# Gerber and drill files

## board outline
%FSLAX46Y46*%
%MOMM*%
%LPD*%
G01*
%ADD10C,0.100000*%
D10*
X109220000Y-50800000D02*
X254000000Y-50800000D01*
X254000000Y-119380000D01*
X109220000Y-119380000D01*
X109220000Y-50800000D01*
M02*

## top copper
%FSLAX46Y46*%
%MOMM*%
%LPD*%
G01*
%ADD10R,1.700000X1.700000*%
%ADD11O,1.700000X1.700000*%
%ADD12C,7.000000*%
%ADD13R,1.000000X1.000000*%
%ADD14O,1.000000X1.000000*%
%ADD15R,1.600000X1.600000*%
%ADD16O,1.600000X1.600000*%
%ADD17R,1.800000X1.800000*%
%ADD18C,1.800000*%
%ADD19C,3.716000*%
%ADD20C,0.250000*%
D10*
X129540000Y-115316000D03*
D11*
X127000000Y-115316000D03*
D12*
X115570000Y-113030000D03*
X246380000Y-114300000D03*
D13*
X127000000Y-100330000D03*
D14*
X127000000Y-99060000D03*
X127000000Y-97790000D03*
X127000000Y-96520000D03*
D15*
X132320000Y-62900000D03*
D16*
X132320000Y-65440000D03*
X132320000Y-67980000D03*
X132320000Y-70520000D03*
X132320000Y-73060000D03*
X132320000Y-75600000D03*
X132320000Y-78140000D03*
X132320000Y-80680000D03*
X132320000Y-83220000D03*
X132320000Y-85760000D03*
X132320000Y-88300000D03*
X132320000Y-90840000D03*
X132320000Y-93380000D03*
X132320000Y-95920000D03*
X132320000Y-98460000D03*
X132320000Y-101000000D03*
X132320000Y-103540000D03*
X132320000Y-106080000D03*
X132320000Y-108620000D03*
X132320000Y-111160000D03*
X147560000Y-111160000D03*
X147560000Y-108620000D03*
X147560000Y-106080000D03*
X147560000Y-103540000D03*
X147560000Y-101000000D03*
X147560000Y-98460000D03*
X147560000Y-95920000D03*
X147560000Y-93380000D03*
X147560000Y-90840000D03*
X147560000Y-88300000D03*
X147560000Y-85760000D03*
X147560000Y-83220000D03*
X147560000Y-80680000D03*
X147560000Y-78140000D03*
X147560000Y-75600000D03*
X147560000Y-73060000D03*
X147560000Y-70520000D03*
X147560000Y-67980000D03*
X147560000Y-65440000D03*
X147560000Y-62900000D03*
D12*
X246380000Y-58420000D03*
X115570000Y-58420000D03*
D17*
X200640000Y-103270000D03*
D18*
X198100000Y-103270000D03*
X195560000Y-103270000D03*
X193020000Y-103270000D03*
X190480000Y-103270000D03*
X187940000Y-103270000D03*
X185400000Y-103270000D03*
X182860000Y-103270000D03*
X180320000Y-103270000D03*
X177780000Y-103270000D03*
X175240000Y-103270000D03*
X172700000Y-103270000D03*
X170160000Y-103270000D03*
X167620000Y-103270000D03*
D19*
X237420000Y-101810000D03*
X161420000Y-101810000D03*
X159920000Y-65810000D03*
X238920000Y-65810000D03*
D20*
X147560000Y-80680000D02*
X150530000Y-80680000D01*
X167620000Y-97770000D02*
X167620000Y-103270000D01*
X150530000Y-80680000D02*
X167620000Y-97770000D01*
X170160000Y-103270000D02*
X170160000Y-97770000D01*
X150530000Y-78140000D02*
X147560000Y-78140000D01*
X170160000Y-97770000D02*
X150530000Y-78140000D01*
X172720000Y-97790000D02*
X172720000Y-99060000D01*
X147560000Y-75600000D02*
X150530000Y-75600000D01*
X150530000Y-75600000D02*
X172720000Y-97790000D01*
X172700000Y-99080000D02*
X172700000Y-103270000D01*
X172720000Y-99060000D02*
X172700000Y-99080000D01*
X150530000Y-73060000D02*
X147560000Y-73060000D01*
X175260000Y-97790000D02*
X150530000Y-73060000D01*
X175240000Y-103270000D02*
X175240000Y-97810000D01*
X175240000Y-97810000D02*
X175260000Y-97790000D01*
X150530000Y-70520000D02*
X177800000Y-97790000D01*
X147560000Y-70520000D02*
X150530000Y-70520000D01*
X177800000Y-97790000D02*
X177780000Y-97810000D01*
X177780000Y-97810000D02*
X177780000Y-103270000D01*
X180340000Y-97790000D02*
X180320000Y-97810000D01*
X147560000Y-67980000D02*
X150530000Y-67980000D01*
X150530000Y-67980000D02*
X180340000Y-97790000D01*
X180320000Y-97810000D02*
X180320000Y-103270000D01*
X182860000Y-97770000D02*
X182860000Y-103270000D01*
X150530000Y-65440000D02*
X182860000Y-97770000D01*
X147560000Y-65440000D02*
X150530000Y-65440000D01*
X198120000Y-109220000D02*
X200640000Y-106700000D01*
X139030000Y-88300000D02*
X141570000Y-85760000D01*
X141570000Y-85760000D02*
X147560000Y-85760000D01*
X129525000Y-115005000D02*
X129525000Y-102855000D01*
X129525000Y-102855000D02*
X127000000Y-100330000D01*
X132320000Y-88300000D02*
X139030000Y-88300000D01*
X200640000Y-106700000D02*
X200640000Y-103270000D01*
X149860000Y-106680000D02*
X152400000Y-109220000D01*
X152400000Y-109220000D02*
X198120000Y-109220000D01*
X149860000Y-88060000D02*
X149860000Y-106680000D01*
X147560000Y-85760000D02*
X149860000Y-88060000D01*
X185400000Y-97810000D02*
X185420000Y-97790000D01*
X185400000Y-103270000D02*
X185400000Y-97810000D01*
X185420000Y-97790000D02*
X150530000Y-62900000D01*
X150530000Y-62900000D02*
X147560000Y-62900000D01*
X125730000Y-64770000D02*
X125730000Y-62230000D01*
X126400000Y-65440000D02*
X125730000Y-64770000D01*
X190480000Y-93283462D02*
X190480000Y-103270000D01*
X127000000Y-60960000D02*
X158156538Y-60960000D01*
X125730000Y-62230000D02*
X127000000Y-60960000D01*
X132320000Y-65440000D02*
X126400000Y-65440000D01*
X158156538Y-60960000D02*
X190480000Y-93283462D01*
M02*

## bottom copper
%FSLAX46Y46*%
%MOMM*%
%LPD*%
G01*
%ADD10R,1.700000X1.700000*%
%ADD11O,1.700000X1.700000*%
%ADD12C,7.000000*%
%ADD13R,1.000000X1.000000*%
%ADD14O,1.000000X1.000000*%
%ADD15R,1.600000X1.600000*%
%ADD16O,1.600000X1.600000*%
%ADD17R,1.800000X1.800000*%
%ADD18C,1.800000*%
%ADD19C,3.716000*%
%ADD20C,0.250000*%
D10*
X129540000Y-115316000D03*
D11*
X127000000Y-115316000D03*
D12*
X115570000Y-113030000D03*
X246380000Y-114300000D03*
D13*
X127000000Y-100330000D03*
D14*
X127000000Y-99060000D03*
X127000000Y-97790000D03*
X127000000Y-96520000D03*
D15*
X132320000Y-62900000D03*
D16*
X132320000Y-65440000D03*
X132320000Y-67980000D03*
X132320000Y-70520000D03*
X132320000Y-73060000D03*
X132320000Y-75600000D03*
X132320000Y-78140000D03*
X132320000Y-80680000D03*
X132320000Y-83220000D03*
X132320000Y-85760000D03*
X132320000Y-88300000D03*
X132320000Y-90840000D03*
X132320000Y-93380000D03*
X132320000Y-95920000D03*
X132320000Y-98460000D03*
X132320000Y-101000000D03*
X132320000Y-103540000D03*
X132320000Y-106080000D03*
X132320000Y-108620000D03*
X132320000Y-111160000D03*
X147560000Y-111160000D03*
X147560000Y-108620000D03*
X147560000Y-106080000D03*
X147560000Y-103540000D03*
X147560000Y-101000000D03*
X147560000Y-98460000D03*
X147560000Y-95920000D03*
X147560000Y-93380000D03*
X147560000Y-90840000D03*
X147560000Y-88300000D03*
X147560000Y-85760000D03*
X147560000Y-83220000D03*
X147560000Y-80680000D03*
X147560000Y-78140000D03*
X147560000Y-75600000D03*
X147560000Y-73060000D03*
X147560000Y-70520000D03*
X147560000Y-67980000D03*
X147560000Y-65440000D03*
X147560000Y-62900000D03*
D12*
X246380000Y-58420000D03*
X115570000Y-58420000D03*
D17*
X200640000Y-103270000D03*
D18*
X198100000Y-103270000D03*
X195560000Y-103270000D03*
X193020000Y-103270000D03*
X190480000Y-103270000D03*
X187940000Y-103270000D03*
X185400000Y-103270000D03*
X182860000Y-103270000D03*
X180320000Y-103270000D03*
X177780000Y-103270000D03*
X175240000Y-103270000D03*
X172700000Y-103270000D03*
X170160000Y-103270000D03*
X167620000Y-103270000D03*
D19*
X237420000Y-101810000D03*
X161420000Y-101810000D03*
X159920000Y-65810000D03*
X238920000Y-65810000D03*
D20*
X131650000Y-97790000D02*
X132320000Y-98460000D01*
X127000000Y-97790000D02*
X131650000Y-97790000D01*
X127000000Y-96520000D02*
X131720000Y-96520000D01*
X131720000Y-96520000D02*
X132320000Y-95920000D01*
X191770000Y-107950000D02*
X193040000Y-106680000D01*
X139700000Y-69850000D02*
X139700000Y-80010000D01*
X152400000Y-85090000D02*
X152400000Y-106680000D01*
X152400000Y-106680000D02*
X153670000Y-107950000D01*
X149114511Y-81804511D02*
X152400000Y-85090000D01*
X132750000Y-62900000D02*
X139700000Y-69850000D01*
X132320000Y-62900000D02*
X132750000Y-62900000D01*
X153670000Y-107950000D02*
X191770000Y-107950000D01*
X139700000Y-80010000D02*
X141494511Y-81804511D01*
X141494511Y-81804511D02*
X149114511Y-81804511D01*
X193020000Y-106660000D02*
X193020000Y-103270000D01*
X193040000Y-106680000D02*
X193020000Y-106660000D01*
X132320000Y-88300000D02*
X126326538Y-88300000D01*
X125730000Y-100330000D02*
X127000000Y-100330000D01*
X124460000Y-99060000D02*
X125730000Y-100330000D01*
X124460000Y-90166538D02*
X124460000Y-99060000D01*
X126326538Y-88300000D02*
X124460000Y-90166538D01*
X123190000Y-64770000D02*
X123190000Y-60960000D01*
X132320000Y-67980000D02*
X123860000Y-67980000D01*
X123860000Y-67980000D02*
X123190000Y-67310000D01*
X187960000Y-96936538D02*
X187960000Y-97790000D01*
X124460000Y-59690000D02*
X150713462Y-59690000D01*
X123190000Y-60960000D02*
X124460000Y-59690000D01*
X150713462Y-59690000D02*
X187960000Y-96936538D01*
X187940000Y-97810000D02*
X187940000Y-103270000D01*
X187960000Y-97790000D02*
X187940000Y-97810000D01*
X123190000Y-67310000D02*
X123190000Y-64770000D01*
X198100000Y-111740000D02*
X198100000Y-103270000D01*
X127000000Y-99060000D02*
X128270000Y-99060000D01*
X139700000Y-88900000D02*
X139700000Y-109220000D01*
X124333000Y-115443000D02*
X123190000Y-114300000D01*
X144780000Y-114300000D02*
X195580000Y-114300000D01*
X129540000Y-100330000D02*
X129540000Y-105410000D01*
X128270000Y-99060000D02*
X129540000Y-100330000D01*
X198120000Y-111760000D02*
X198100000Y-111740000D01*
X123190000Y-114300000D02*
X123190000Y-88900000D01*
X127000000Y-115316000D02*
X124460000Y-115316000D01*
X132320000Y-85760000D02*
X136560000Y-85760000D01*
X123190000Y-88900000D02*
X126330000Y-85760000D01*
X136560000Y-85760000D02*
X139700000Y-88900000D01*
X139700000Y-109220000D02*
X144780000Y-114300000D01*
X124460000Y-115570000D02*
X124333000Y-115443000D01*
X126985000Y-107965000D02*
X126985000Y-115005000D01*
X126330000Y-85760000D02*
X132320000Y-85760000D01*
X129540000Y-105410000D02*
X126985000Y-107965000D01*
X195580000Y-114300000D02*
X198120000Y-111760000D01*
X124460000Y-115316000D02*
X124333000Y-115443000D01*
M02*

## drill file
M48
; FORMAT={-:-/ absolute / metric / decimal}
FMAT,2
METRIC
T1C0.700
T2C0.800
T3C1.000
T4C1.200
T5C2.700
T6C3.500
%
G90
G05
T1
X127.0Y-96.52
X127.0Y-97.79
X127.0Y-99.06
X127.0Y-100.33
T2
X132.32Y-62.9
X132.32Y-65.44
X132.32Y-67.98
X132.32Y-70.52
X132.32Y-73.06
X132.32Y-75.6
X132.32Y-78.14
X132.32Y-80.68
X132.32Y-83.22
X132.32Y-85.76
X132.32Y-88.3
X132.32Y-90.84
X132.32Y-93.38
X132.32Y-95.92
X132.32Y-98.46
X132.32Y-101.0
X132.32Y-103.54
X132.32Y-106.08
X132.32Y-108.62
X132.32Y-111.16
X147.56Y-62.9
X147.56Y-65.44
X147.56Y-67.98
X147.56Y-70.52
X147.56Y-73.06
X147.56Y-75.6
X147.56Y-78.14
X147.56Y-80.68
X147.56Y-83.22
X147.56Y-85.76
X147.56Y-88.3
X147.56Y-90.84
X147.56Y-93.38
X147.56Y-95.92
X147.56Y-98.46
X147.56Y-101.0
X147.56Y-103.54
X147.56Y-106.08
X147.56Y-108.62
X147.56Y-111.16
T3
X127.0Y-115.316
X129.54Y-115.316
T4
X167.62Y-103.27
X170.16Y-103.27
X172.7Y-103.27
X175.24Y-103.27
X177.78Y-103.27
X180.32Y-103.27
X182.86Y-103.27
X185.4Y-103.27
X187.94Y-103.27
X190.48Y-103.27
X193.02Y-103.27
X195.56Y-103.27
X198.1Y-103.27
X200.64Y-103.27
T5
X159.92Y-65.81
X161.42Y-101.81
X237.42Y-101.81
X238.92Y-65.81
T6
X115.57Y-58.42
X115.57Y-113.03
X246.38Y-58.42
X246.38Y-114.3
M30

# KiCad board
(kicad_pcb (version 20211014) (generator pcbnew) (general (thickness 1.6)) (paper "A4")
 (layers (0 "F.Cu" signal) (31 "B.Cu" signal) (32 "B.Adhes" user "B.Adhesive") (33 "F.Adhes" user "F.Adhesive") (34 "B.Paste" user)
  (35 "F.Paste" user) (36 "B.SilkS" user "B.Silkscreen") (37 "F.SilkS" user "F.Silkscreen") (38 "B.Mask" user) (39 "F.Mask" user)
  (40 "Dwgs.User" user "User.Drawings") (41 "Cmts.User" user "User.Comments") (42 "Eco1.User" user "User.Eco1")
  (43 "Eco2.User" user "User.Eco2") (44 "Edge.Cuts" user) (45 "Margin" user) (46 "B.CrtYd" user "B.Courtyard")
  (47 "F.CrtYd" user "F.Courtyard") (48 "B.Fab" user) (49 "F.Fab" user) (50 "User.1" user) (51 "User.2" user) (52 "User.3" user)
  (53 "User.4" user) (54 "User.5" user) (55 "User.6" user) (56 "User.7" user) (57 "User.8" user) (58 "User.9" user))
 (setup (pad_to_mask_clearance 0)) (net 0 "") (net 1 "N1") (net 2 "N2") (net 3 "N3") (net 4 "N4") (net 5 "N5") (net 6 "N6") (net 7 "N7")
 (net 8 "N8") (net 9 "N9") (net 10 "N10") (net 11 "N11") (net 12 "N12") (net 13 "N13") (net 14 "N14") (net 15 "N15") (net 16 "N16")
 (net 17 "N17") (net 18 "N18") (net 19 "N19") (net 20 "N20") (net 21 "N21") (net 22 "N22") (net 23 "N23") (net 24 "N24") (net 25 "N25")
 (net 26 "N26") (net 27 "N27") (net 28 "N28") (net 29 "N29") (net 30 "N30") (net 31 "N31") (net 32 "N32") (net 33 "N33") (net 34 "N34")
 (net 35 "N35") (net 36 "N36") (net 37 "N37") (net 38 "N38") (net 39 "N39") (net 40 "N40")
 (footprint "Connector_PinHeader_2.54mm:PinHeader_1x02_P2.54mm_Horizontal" (layer "F.Cu") (at 129.54 115.316 -90)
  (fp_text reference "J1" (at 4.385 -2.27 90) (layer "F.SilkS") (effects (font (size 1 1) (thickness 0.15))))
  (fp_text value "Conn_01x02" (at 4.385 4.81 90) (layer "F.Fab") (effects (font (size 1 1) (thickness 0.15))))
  (pad "1" thru_hole rect (at 0 0 270) (size 1.7 1.7) (drill 1) (layers *.Cu *.Mask) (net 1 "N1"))
  (pad "2" thru_hole oval (at 0 2.54 270) (size 1.7 1.7) (drill 1) (layers *.Cu *.Mask) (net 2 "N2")))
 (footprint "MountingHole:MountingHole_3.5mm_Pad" (layer "F.Cu") (at 115.57 113.03)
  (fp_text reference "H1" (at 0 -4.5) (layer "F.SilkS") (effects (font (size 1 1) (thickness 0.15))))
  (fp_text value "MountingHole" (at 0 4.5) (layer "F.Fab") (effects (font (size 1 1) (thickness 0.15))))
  (pad "1" thru_hole circle (at 0 0) (size 7 7) (drill 3.5) (layers *.Cu *.Mask)))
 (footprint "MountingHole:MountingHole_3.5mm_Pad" (layer "F.Cu") (at 246.38 114.3)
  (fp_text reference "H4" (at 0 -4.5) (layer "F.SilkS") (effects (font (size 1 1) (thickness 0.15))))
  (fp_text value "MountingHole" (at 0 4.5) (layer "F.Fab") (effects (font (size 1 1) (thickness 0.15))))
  (pad "1" thru_hole circle (at 0 0) (size 7 7) (drill 3.5) (layers *.Cu *.Mask)))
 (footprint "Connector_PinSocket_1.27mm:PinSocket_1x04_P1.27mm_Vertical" (layer "F.Cu") (at 127 100.33 180)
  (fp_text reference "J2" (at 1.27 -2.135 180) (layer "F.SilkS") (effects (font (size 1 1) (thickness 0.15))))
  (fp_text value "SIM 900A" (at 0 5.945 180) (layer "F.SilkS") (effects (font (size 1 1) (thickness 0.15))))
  (pad "1" thru_hole rect (at 0 0 180) (size 1 1) (drill 0.7) (layers *.Cu *.Mask) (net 1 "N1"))
  (pad "2" thru_hole oval (at 0 1.27 180) (size 1 1) (drill 0.7) (layers *.Cu *.Mask) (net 2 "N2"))
  (pad "3" thru_hole oval (at 0 2.54 180) (size 1 1) (drill 0.7) (layers *.Cu *.Mask) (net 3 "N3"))
  (pad "4" thru_hole oval (at 0 3.81 180) (size 1 1) (drill 0.7) (layers *.Cu *.Mask) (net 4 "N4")))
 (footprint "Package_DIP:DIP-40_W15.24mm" (layer "F.Cu") (at 132.32 62.9)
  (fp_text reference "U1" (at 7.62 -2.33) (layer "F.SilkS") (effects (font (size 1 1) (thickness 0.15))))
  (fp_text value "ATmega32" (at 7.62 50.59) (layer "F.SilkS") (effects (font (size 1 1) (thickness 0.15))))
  (pad "1" thru_hole rect (at 0 0) (size 1.6 1.6) (drill 0.8) (layers *.Cu *.Mask) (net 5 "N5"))
  (pad "2" thru_hole oval (at 0 2.54) (size 1.6 1.6) (drill 0.8) (layers *.Cu *.Mask) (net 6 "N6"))
  (pad "3" thru_hole oval (at 0 5.08) (size 1.6 1.6) (drill 0.8) (layers *.Cu *.Mask) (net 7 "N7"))
  (pad "4" thru_hole oval (at 0 7.62) (size 1.6 1.6) (drill 0.8) (layers *.Cu *.Mask) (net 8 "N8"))
  (pad "5" thru_hole oval (at 0 10.16) (size 1.6 1.6) (drill 0.8) (layers *.Cu *.Mask) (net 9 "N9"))
  (pad "6" thru_hole oval (at 0 12.7) (size 1.6 1.6) (drill 0.8) (layers *.Cu *.Mask) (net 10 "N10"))
  (pad "7" thru_hole oval (at 0 15.24) (size 1.6 1.6) (drill 0.8) (layers *.Cu *.Mask) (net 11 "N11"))
  (pad "8" thru_hole oval (at 0 17.78) (size 1.6 1.6) (drill 0.8) (layers *.Cu *.Mask) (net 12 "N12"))
  (pad "9" thru_hole oval (at 0 20.32) (size 1.6 1.6) (drill 0.8) (layers *.Cu *.Mask) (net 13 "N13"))
  (pad "10" thru_hole oval (at 0 22.86) (size 1.6 1.6) (drill 0.8) (layers *.Cu *.Mask) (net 2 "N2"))
  (pad "11" thru_hole oval (at 0 25.4) (size 1.6 1.6) (drill 0.8) (layers *.Cu *.Mask) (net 1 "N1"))
  (pad "12" thru_hole oval (at 0 27.94) (size 1.6 1.6) (drill 0.8) (layers *.Cu *.Mask) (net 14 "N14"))
  (pad "13" thru_hole oval (at 0 30.48) (size 1.6 1.6) (drill 0.8) (layers *.Cu *.Mask) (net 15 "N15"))
  (pad "14" thru_hole oval (at 0 33.02) (size 1.6 1.6) (drill 0.8) (layers *.Cu *.Mask) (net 4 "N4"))
  (pad "15" thru_hole oval (at 0 35.56) (size 1.6 1.6) (drill 0.8) (layers *.Cu *.Mask) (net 3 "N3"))
  (pad "16" thru_hole oval (at 0 38.1) (size 1.6 1.6) (drill 0.8) (layers *.Cu *.Mask) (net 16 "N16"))
  (pad "17" thru_hole oval (at 0 40.64) (size 1.6 1.6) (drill 0.8) (layers *.Cu *.Mask) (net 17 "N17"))
  (pad "18" thru_hole oval (at 0 43.18) (size 1.6 1.6) (drill 0.8) (layers *.Cu *.Mask) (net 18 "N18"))
  (pad "19" thru_hole oval (at 0 45.72) (size 1.6 1.6) (drill 0.8) (layers *.Cu *.Mask) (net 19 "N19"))
  (pad "20" thru_hole oval (at 0 48.26) (size 1.6 1.6) (drill 0.8) (layers *.Cu *.Mask) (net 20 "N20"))
  (pad "21" thru_hole oval (at 15.24 48.26) (size 1.6 1.6) (drill 0.8) (layers *.Cu *.Mask) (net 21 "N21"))
  (pad "22" thru_hole oval (at 15.24 45.72) (size 1.6 1.6) (drill 0.8) (layers *.Cu *.Mask) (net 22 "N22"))
  (pad "23" thru_hole oval (at 15.24 43.18) (size 1.6 1.6) (drill 0.8) (layers *.Cu *.Mask) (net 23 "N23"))
  (pad "24" thru_hole oval (at 15.24 40.64) (size 1.6 1.6) (drill 0.8) (layers *.Cu *.Mask) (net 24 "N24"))
  (pad "25" thru_hole oval (at 15.24 38.1) (size 1.6 1.6) (drill 0.8) (layers *.Cu *.Mask) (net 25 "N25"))
  (pad "26" thru_hole oval (at 15.24 35.56) (size 1.6 1.6) (drill 0.8) (layers *.Cu *.Mask) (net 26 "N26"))
  (pad "27" thru_hole oval (at 15.24 33.02) (size 1.6 1.6) (drill 0.8) (layers *.Cu *.Mask) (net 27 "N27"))
  (pad "28" thru_hole oval (at 15.24 30.48) (size 1.6 1.6) (drill 0.8) (layers *.Cu *.Mask) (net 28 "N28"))
  (pad "29" thru_hole oval (at 15.24 27.94) (size 1.6 1.6) (drill 0.8) (layers *.Cu *.Mask) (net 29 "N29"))
  (pad "30" thru_hole oval (at 15.24 25.4) (size 1.6 1.6) (drill 0.8) (layers *.Cu *.Mask) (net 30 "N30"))
  (pad "31" thru_hole oval (at 15.24 22.86) (size 1.6 1.6) (drill 0.8) (layers *.Cu *.Mask) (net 1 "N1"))
  (pad "32" thru_hole oval (at 15.24 20.32) (size 1.6 1.6) (drill 0.8) (layers *.Cu *.Mask) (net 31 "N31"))
  (pad "33" thru_hole oval (at 15.24 17.78) (size 1.6 1.6) (drill 0.8) (layers *.Cu *.Mask) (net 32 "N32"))
  (pad "34" thru_hole oval (at 15.24 15.24) (size 1.6 1.6) (drill 0.8) (layers *.Cu *.Mask) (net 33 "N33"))
  (pad "35" thru_hole oval (at 15.24 12.7) (size 1.6 1.6) (drill 0.8) (layers *.Cu *.Mask) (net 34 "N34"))
  (pad "36" thru_hole oval (at 15.24 10.16) (size 1.6 1.6) (drill 0.8) (layers *.Cu *.Mask) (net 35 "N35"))
  (pad "37" thru_hole oval (at 15.24 7.62) (size 1.6 1.6) (drill 0.8) (layers *.Cu *.Mask) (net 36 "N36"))
  (pad "38" thru_hole oval (at 15.24 5.08) (size 1.6 1.6) (drill 0.8) (layers *.Cu *.Mask) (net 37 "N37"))
  (pad "39" thru_hole oval (at 15.24 2.54) (size 1.6 1.6) (drill 0.8) (layers *.Cu *.Mask) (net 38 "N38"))
  (pad "40" thru_hole oval (at 15.24 0) (size 1.6 1.6) (drill 0.8) (layers *.Cu *.Mask) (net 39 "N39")))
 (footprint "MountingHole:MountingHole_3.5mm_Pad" (layer "F.Cu") (at 246.38 58.42)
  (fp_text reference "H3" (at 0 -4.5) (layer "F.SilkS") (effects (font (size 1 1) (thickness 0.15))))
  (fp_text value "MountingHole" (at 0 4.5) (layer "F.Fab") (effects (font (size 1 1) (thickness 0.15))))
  (pad "1" thru_hole circle (at 0 0) (size 7 7) (drill 3.5) (layers *.Cu *.Mask)))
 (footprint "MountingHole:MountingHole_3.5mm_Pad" (layer "F.Cu") (at 115.57 58.42)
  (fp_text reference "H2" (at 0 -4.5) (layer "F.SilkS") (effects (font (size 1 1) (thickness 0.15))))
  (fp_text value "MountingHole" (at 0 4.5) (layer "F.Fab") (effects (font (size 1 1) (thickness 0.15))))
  (pad "1" thru_hole circle (at 0 0) (size 7 7) (drill 3.5) (layers *.Cu *.Mask)))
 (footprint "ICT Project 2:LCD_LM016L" (layer "F.Cu") (at 200.64 103.27)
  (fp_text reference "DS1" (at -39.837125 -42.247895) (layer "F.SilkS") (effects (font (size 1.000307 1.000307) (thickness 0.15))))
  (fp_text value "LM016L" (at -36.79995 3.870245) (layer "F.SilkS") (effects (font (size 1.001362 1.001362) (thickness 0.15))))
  (pad "1" thru_hole rect locked (at 0 0) (size 1.8 1.8) (drill 1.2) (layers *.Cu *.Mask) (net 1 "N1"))
  (pad "2" thru_hole circle locked (at -2.54 0) (size 1.8 1.8) (drill 1.2) (layers *.Cu *.Mask) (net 2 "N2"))
  (pad "3" thru_hole circle locked (at -5.08 0) (size 1.8 1.8) (drill 1.2) (layers *.Cu *.Mask) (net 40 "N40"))
  (pad "4" thru_hole circle locked (at -7.62 0) (size 1.8 1.8) (drill 1.2) (layers *.Cu *.Mask) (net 5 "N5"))
  (pad "5" thru_hole circle locked (at -10.16 0) (size 1.8 1.8) (drill 1.2) (layers *.Cu *.Mask) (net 6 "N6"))
  (pad "6" thru_hole circle locked (at -12.7 0) (size 1.8 1.8) (drill 1.2) (layers *.Cu *.Mask) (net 7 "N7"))
  (pad "7" thru_hole circle locked (at -15.24 0) (size 1.8 1.8) (drill 1.2) (layers *.Cu *.Mask) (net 39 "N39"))
  (pad "8" thru_hole circle locked (at -17.78 0) (size 1.8 1.8) (drill 1.2) (layers *.Cu *.Mask) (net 38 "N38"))
  (pad "9" thru_hole circle locked (at -20.32 0) (size 1.8 1.8) (drill 1.2) (layers *.Cu *.Mask) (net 37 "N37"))
  (pad "10" thru_hole circle locked (at -22.86 0) (size 1.8 1.8) (drill 1.2) (layers *.Cu *.Mask) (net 36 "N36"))
  (pad "11" thru_hole circle locked (at -25.4 0) (size 1.8 1.8) (drill 1.2) (layers *.Cu *.Mask) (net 35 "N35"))
  (pad "12" thru_hole circle locked (at -27.94 0) (size 1.8 1.8) (drill 1.2) (layers *.Cu *.Mask) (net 34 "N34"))
  (pad "13" thru_hole circle locked (at -30.48 0) (size 1.8 1.8) (drill 1.2) (layers *.Cu *.Mask) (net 33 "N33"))
  (pad "14" thru_hole circle locked (at -33.02 0) (size 1.8 1.8) (drill 1.2) (layers *.Cu *.Mask) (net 32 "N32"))
  (pad "15" thru_hole circle locked (at 36.78 -1.46) (size 3.716 3.716) (drill 2.7) (layers *.Cu *.Mask))
  (pad "16" thru_hole circle locked (at -39.22 -1.46) (size 3.716 3.716) (drill 2.7) (layers *.Cu *.Mask))
  (pad "17" thru_hole circle locked (at -40.72 -37.46) (size 3.716 3.716) (drill 2.7) (layers *.Cu *.Mask))
  (pad "18" thru_hole circle locked (at 38.28 -37.46) (size 3.716 3.716) (drill 2.7) (layers *.Cu *.Mask)))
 (gr_rect (start 109.22 50.8) (end 254 119.38) (layer "Edge.Cuts") (width 0.1) (fill none))
 (segment (start 131.65 97.79) (end 132.32 98.46) (width 0.25) (layer "B.Cu") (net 3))
 (segment (start 127 97.79) (end 131.65 97.79) (width 0.25) (layer "B.Cu") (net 3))
 (segment (start 127 96.52) (end 131.72 96.52) (width 0.25) (layer "B.Cu") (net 4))
 (segment (start 131.72 96.52) (end 132.32 95.92) (width 0.25) (layer "B.Cu") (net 4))
 (segment (start 191.77 107.95) (end 193.04 106.68) (width 0.25) (layer "B.Cu") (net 5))
 (segment (start 139.7 69.85) (end 139.7 80.01) (width 0.25) (layer "B.Cu") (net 5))
 (segment (start 152.4 85.09) (end 152.4 106.68) (width 0.25) (layer "B.Cu") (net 5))
 (segment (start 152.4 106.68) (end 153.67 107.95) (width 0.25) (layer "B.Cu") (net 5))
 (segment (start 149.114511 81.804511) (end 152.4 85.09) (width 0.25) (layer "B.Cu") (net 5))
 (segment (start 132.75 62.9) (end 139.7 69.85) (width 0.25) (layer "B.Cu") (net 5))
 (segment (start 132.32 62.9) (end 132.75 62.9) (width 0.25) (layer "B.Cu") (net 5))
 (segment (start 153.67 107.95) (end 191.77 107.95) (width 0.25) (layer "B.Cu") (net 5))
 (segment (start 139.7 80.01) (end 141.494511 81.804511) (width 0.25) (layer "B.Cu") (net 5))
 (segment (start 141.494511 81.804511) (end 149.114511 81.804511) (width 0.25) (layer "B.Cu") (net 5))
 (segment (start 193.02 106.66) (end 193.02 103.27) (width 0.25) (layer "B.Cu") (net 5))
 (segment (start 193.04 106.68) (end 193.02 106.66) (width 0.25) (layer "B.Cu") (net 5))
 (segment (start 147.56 80.68) (end 150.53 80.68) (width 0.25) (layer "F.Cu") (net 32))
 (segment (start 167.62 97.77) (end 167.62 103.27) (width 0.25) (layer "F.Cu") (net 32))
 (segment (start 150.53 80.68) (end 167.62 97.77) (width 0.25) (layer "F.Cu") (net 32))
 (segment (start 170.16 103.27) (end 170.16 97.77) (width 0.25) (layer "F.Cu") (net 33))
 (segment (start 150.53 78.14) (end 147.56 78.14) (width 0.25) (layer "F.Cu") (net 33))
 (segment (start 170.16 97.77) (end 150.53 78.14) (width 0.25) (layer "F.Cu") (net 33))
 (segment (start 172.72 97.79) (end 172.72 99.06) (width 0.25) (layer "F.Cu") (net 34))
 (segment (start 147.56 75.6) (end 150.53 75.6) (width 0.25) (layer "F.Cu") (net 34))
 (segment (start 150.53 75.6) (end 172.72 97.79) (width 0.25) (layer "F.Cu") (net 34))
 (segment (start 172.7 99.08) (end 172.7 103.27) (width 0.25) (layer "F.Cu") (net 34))
 (segment (start 172.72 99.06) (end 172.7 99.08) (width 0.25) (layer "F.Cu") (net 34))
 (segment (start 150.53 73.06) (end 147.56 73.06) (width 0.25) (layer "F.Cu") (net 35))
 (segment (start 175.26 97.79) (end 150.53 73.06) (width 0.25) (layer "F.Cu") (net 35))
 (segment (start 175.24 103.27) (end 175.24 97.81) (width 0.25) (layer "F.Cu") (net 35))
 (segment (start 175.24 97.81) (end 175.26 97.79) (width 0.25) (layer "F.Cu") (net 35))
 (segment (start 150.53 70.52) (end 177.8 97.79) (width 0.25) (layer "F.Cu") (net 36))
 (segment (start 147.56 70.52) (end 150.53 70.52) (width 0.25) (layer "F.Cu") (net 36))
 (segment (start 177.8 97.79) (end 177.78 97.81) (width 0.25) (layer "F.Cu") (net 36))
 (segment (start 177.78 97.81) (end 177.78 103.27) (width 0.25) (layer "F.Cu") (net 36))
 (segment (start 180.34 97.79) (end 180.32 97.81) (width 0.25) (layer "F.Cu") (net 37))
 (segment (start 147.56 67.98) (end 150.53 67.98) (width 0.25) (layer "F.Cu") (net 37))
 (segment (start 150.53 67.98) (end 180.34 97.79) (width 0.25) (layer "F.Cu") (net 37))
 (segment (start 180.32 97.81) (end 180.32 103.27) (width 0.25) (layer "F.Cu") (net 37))
 (segment (start 182.86 97.77) (end 182.86 103.27) (width 0.25) (layer "F.Cu") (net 38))
 (segment (start 150.53 65.44) (end 182.86 97.77) (width 0.25) (layer "F.Cu") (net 38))
 (segment (start 147.56 65.44) (end 150.53 65.44) (width 0.25) (layer "F.Cu") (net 38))
 (segment (start 198.12 109.22) (end 200.64 106.7) (width 0.25) (layer "F.Cu") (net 1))
 (segment (start 139.03 88.3) (end 141.57 85.76) (width 0.25) (layer "F.Cu") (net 1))
 (segment (start 141.57 85.76) (end 147.56 85.76) (width 0.25) (layer "F.Cu") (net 1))
 (segment (start 129.525 115.005) (end 129.525 102.855) (width 0.25) (layer "F.Cu") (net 1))
 (segment (start 129.525 102.855) (end 127 100.33) (width 0.25) (layer "F.Cu") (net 1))
 (segment (start 132.32 88.3) (end 139.03 88.3) (width 0.25) (layer "F.Cu") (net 1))
 (segment (start 200.64 106.7) (end 200.64 103.27) (width 0.25) (layer "F.Cu") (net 1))
 (segment (start 149.86 106.68) (end 152.4 109.22) (width 0.25) (layer "F.Cu") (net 1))
 (segment (start 152.4 109.22) (end 198.12 109.22) (width 0.25) (layer "F.Cu") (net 1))
 (segment (start 149.86 88.06) (end 149.86 106.68) (width 0.25) (layer "F.Cu") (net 1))
 (segment (start 147.56 85.76) (end 149.86 88.06) (width 0.25) (layer "F.Cu") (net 1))
 (segment (start 132.32 88.3) (end 126.326538 88.3) (width 0.25) (layer "B.Cu") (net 1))
 (segment (start 125.73 100.33) (end 127 100.33) (width 0.25) (layer "B.Cu") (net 1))
 (segment (start 124.46 99.06) (end 125.73 100.33) (width 0.25) (layer "B.Cu") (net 1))
 (segment (start 124.46 90.166538) (end 124.46 99.06) (width 0.25) (layer "B.Cu") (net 1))
 (segment (start 126.326538 88.3) (end 124.46 90.166538) (width 0.25) (layer "B.Cu") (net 1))
 (segment (start 185.4 97.81) (end 185.42 97.79) (width 0.25) (layer "F.Cu") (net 39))
 (segment (start 185.4 103.27) (end 185.4 97.81) (width 0.25) (layer "F.Cu") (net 39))
 (segment (start 185.42 97.79) (end 150.53 62.9) (width 0.25) (layer "F.Cu") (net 39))
 (segment (start 150.53 62.9) (end 147.56 62.9) (width 0.25) (layer "F.Cu") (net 39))
 (segment (start 125.73 64.77) (end 125.73 62.23) (width 0.25) (layer "F.Cu") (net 6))
 (segment (start 126.4 65.44) (end 125.73 64.77) (width 0.25) (layer "F.Cu") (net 6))
 (segment (start 190.48 93.283462) (end 190.48 103.27) (width 0.25) (layer "F.Cu") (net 6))
 (segment (start 127 60.96) (end 158.156538 60.96) (width 0.25) (layer "F.Cu") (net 6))
 (segment (start 125.73 62.23) (end 127 60.96) (width 0.25) (layer "F.Cu") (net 6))
 (segment (start 132.32 65.44) (end 126.4 65.44) (width 0.25) (layer "F.Cu") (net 6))
 (segment (start 158.156538 60.96) (end 190.48 93.283462) (width 0.25) (layer "F.Cu") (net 6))
 (segment (start 123.19 64.77) (end 123.19 60.96) (width 0.25) (layer "B.Cu") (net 7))
 (segment (start 132.32 67.98) (end 123.86 67.98) (width 0.25) (layer "B.Cu") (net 7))
 (segment (start 123.86 67.98) (end 123.19 67.31) (width 0.25) (layer "B.Cu") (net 7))
 (segment (start 187.96 96.936538) (end 187.96 97.79) (width 0.25) (layer "B.Cu") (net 7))
 (segment (start 124.46 59.69) (end 150.713462 59.69) (width 0.25) (layer "B.Cu") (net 7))
 (segment (start 123.19 60.96) (end 124.46 59.69) (width 0.25) (layer "B.Cu") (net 7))
 (segment (start 150.713462 59.69) (end 187.96 96.936538) (width 0.25) (layer "B.Cu") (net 7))
 (segment (start 187.94 97.81) (end 187.94 103.27) (width 0.25) (layer "B.Cu") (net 7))
 (segment (start 187.96 97.79) (end 187.94 97.81) (width 0.25) (layer "B.Cu") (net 7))
 (segment (start 123.19 67.31) (end 123.19 64.77) (width 0.25) (layer "B.Cu") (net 7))
 (segment (start 198.1 111.74) (end 198.1 103.27) (width 0.25) (layer "B.Cu") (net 2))
 (segment (start 127 99.06) (end 128.27 99.06) (width 0.25) (layer "B.Cu") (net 2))
 (segment (start 139.7 88.9) (end 139.7 109.22) (width 0.25) (layer "B.Cu") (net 2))
 (segment (start 124.333 115.443) (end 123.19 114.3) (width 0.25) (layer "B.Cu") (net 2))
 (segment (start 144.78 114.3) (end 195.58 114.3) (width 0.25) (layer "B.Cu") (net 2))
 (segment (start 129.54 100.33) (end 129.54 105.41) (width 0.25) (layer "B.Cu") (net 2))
 (segment (start 128.27 99.06) (end 129.54 100.33) (width 0.25) (layer "B.Cu") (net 2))
 (segment (start 198.12 111.76) (end 198.1 111.74) (width 0.25) (layer "B.Cu") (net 2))
 (segment (start 123.19 114.3) (end 123.19 88.9) (width 0.25) (layer "B.Cu") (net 2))
 (segment (start 127 115.316) (end 124.46 115.316) (width 0.25) (layer "B.Cu") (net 2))
 (segment (start 132.32 85.76) (end 136.56 85.76) (width 0.25) (layer "B.Cu") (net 2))
 (segment (start 123.19 88.9) (end 126.33 85.76) (width 0.25) (layer "B.Cu") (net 2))
 (segment (start 136.56 85.76) (end 139.7 88.9) (width 0.25) (layer "B.Cu") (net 2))
 (segment (start 139.7 109.22) (end 144.78 114.3) (width 0.25) (layer "B.Cu") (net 2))
 (segment (start 124.46 115.57) (end 124.333 115.443) (width 0.25) (layer "B.Cu") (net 2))
 (segment (start 126.985 107.965) (end 126.985 115.005) (width 0.25) (layer "B.Cu") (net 2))
 (segment (start 126.33 85.76) (end 132.32 85.76) (width 0.25) (layer "B.Cu") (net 2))
 (segment (start 129.54 105.41) (end 126.985 107.965) (width 0.25) (layer "B.Cu") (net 2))
 (segment (start 195.58 114.3) (end 198.12 111.76) (width 0.25) (layer "B.Cu") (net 2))
 (segment (start 124.46 115.316) (end 124.333 115.443) (width 0.25) (layer "B.Cu") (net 2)))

